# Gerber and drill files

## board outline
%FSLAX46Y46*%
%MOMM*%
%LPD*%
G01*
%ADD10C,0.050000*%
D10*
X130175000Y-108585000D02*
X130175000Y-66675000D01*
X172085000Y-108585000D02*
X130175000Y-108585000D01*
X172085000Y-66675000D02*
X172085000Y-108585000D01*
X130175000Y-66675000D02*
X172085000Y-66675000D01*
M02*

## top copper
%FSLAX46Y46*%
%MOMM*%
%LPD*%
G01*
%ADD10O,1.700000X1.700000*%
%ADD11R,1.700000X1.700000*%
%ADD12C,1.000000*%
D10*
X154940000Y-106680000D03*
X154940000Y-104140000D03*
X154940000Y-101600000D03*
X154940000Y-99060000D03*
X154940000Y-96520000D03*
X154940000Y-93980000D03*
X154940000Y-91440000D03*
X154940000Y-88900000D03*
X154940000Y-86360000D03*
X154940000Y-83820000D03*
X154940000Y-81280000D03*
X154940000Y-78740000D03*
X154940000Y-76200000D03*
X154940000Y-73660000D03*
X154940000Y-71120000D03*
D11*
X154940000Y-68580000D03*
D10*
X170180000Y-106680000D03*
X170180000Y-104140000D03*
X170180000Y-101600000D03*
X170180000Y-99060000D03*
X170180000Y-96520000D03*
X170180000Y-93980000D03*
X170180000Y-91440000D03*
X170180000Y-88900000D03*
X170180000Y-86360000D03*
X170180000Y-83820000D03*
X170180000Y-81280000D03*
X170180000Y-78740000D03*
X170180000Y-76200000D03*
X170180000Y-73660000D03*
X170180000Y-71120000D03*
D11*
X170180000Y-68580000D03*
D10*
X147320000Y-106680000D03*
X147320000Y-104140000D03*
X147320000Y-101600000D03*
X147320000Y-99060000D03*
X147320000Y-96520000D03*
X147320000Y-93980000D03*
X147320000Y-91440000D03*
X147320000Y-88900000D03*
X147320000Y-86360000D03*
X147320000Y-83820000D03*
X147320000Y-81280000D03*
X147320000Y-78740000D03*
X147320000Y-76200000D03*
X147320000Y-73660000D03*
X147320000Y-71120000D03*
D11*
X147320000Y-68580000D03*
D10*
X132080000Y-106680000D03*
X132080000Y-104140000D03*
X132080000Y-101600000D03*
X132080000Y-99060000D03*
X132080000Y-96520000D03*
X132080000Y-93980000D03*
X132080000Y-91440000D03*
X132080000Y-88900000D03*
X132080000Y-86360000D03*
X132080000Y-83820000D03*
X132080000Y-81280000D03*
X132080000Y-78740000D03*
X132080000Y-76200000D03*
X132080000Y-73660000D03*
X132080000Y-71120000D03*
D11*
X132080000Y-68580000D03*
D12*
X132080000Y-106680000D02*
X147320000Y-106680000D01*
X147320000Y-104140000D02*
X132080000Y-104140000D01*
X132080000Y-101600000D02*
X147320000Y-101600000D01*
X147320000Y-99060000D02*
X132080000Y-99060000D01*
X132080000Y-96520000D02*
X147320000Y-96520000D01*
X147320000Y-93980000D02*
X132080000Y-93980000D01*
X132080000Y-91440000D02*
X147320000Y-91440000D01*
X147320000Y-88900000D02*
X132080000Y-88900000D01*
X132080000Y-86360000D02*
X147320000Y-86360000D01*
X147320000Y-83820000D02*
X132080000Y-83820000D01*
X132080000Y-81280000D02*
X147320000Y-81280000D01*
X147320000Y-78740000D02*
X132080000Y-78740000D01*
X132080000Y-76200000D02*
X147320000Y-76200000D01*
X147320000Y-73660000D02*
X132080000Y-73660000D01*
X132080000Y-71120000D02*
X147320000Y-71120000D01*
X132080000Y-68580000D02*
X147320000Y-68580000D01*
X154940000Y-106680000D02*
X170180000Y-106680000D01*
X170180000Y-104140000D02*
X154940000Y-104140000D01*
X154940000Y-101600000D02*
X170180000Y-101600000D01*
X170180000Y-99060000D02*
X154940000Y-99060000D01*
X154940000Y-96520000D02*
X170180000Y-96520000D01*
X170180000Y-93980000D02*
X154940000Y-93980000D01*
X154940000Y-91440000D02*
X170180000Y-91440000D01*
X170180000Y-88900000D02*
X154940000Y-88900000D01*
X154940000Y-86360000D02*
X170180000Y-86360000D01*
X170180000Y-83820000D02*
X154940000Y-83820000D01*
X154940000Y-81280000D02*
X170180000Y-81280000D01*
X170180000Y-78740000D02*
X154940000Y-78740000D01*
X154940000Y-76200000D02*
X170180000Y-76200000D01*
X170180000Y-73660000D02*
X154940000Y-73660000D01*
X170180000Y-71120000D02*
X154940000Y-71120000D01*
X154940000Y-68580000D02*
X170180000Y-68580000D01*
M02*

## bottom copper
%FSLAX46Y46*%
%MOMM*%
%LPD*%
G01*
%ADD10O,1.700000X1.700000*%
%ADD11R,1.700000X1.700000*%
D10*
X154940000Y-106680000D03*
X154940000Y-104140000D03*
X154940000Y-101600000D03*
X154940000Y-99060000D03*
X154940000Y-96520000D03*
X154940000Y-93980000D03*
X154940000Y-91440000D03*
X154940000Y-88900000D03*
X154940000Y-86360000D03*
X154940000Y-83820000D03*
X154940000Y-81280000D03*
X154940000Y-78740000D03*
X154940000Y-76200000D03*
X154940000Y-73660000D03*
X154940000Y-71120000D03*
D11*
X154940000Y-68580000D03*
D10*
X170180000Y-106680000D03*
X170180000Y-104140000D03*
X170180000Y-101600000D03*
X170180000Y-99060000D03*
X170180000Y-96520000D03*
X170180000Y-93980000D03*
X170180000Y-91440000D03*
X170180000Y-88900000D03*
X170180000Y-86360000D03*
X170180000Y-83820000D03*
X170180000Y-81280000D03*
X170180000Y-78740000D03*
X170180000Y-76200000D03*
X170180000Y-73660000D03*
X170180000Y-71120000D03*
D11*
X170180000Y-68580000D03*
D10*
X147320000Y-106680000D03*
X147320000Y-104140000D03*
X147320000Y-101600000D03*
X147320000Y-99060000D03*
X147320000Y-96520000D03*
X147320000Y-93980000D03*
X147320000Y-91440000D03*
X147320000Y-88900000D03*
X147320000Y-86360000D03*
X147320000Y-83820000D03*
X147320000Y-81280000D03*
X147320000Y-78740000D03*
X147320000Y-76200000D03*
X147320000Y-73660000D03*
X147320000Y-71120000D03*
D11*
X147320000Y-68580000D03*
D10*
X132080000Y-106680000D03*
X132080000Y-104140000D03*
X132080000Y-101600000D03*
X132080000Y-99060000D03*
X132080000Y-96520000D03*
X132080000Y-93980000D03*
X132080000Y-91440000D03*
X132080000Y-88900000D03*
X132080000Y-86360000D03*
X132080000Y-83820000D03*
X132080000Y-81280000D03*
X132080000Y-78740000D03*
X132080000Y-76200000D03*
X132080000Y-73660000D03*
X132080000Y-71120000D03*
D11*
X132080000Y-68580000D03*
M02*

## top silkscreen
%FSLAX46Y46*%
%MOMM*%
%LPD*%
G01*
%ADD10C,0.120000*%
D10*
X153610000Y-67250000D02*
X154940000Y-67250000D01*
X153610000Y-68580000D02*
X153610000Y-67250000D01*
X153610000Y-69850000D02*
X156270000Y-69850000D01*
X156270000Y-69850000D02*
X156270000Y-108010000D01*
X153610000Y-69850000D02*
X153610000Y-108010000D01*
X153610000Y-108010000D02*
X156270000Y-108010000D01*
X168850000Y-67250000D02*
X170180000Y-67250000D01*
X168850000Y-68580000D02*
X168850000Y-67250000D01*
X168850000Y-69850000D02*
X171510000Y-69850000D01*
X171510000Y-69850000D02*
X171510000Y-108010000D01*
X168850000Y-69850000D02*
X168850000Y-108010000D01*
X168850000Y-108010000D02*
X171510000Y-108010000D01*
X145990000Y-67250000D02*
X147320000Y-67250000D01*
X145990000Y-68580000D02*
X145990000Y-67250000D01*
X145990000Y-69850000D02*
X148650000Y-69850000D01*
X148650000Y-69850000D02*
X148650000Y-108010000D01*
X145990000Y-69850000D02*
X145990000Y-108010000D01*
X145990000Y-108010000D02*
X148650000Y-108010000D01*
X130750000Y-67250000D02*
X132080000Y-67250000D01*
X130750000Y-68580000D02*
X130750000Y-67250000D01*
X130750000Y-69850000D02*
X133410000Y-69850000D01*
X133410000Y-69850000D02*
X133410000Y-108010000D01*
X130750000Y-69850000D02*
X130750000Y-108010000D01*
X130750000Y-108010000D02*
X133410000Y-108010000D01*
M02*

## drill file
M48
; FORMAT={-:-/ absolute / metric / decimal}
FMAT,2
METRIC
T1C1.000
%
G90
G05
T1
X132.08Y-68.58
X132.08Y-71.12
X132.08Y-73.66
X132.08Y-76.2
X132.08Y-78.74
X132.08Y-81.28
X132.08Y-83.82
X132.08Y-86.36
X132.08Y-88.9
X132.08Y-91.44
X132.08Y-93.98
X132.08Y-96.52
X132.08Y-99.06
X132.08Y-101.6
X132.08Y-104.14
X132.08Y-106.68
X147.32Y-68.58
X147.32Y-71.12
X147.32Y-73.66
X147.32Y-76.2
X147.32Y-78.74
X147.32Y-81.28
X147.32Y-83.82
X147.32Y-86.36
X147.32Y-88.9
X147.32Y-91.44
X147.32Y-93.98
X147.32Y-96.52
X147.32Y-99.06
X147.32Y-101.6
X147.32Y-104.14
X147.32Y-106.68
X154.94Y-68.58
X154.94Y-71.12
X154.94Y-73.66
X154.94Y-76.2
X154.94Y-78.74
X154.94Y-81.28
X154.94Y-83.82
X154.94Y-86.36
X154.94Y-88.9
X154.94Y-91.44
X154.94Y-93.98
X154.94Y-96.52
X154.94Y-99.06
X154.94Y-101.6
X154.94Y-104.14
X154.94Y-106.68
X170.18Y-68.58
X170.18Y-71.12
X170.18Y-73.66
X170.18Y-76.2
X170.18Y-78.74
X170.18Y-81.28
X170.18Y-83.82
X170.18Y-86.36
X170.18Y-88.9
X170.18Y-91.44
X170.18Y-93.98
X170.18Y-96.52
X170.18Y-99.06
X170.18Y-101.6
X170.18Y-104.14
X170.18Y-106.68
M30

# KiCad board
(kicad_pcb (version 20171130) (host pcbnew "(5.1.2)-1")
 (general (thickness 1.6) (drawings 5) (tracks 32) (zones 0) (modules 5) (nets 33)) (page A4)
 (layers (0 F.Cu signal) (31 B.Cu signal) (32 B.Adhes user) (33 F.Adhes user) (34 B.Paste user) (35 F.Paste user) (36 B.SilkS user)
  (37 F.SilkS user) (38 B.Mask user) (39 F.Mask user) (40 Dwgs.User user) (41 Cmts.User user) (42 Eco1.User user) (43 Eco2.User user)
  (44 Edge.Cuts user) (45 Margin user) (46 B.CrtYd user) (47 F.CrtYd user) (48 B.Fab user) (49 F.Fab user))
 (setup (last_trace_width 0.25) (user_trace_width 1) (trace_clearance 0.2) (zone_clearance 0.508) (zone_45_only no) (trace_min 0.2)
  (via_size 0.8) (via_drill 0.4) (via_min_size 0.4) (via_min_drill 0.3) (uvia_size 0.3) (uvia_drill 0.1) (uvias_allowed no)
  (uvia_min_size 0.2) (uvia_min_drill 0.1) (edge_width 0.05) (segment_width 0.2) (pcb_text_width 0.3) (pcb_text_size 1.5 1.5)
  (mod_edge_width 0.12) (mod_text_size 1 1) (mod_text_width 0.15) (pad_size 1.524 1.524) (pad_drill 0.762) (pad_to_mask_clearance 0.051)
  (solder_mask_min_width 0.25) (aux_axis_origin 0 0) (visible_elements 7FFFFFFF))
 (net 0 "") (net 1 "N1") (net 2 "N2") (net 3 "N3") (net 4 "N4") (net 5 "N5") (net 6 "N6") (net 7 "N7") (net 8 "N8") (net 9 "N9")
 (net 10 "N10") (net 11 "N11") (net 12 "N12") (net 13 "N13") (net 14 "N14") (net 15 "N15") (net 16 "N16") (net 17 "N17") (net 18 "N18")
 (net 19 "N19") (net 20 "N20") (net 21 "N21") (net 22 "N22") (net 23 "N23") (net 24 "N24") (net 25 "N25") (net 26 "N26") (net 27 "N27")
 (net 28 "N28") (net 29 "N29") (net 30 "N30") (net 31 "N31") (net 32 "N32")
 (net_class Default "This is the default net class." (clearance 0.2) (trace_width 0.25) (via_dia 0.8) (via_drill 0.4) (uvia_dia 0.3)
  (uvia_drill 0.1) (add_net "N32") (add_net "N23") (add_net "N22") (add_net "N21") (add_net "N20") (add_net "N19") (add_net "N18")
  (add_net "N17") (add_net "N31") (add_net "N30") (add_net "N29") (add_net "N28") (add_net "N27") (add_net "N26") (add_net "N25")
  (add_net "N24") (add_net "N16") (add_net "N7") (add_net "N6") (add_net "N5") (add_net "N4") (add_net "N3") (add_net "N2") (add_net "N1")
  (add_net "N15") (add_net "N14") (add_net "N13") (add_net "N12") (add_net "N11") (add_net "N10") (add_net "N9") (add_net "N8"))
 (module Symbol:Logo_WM (layer B.Cu) (at 161.925 83.82 90)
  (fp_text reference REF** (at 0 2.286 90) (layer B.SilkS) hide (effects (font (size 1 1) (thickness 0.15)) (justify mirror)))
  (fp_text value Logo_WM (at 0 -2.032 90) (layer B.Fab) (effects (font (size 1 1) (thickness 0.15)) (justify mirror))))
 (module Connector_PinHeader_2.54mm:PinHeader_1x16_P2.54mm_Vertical (layer F.Cu) (at 154.94 68.58)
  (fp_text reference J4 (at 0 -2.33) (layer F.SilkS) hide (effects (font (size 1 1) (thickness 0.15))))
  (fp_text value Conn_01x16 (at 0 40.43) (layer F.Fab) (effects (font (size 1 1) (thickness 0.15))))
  (fp_line (start -1.33 -1.33) (end 0 -1.33) (layer F.SilkS) (width 0.12))
  (fp_line (start -1.33 0) (end -1.33 -1.33) (layer F.SilkS) (width 0.12))
  (fp_line (start -1.33 1.27) (end 1.33 1.27) (layer F.SilkS) (width 0.12))
  (fp_line (start 1.33 1.27) (end 1.33 39.43) (layer F.SilkS) (width 0.12))
  (fp_line (start -1.33 1.27) (end -1.33 39.43) (layer F.SilkS) (width 0.12))
  (fp_line (start -1.33 39.43) (end 1.33 39.43) (layer F.SilkS) (width 0.12))
  (pad 16 thru_hole oval (at 0 38.1) (size 1.7 1.7) (drill 1) (layers *.Cu *.Mask) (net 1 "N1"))
  (pad 15 thru_hole oval (at 0 35.56) (size 1.7 1.7) (drill 1) (layers *.Cu *.Mask) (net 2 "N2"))
  (pad 14 thru_hole oval (at 0 33.02) (size 1.7 1.7) (drill 1) (layers *.Cu *.Mask) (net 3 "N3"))
  (pad 13 thru_hole oval (at 0 30.48) (size 1.7 1.7) (drill 1) (layers *.Cu *.Mask) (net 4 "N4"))
  (pad 12 thru_hole oval (at 0 27.94) (size 1.7 1.7) (drill 1) (layers *.Cu *.Mask) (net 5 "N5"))
  (pad 11 thru_hole oval (at 0 25.4) (size 1.7 1.7) (drill 1) (layers *.Cu *.Mask) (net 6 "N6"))
  (pad 10 thru_hole oval (at 0 22.86) (size 1.7 1.7) (drill 1) (layers *.Cu *.Mask) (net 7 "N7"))
  (pad 9 thru_hole oval (at 0 20.32) (size 1.7 1.7) (drill 1) (layers *.Cu *.Mask) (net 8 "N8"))
  (pad 8 thru_hole oval (at 0 17.78) (size 1.7 1.7) (drill 1) (layers *.Cu *.Mask) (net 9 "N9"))
  (pad 7 thru_hole oval (at 0 15.24) (size 1.7 1.7) (drill 1) (layers *.Cu *.Mask) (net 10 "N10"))
  (pad 6 thru_hole oval (at 0 12.7) (size 1.7 1.7) (drill 1) (layers *.Cu *.Mask) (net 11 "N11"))
  (pad 5 thru_hole oval (at 0 10.16) (size 1.7 1.7) (drill 1) (layers *.Cu *.Mask) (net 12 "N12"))
  (pad 4 thru_hole oval (at 0 7.62) (size 1.7 1.7) (drill 1) (layers *.Cu *.Mask) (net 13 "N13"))
  (pad 3 thru_hole oval (at 0 5.08) (size 1.7 1.7) (drill 1) (layers *.Cu *.Mask) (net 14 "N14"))
  (pad 2 thru_hole oval (at 0 2.54) (size 1.7 1.7) (drill 1) (layers *.Cu *.Mask) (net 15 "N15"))
  (pad 1 thru_hole rect (at 0 0) (size 1.7 1.7) (drill 1) (layers *.Cu *.Mask) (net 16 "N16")))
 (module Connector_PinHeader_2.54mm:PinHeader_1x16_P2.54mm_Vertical (layer F.Cu) (at 170.18 68.58)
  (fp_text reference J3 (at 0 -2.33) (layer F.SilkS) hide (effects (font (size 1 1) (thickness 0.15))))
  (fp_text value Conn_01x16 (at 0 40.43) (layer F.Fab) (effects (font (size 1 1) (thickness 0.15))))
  (fp_line (start -1.33 -1.33) (end 0 -1.33) (layer F.SilkS) (width 0.12))
  (fp_line (start -1.33 0) (end -1.33 -1.33) (layer F.SilkS) (width 0.12))
  (fp_line (start -1.33 1.27) (end 1.33 1.27) (layer F.SilkS) (width 0.12))
  (fp_line (start 1.33 1.27) (end 1.33 39.43) (layer F.SilkS) (width 0.12))
  (fp_line (start -1.33 1.27) (end -1.33 39.43) (layer F.SilkS) (width 0.12))
  (fp_line (start -1.33 39.43) (end 1.33 39.43) (layer F.SilkS) (width 0.12))
  (pad 16 thru_hole oval (at 0 38.1) (size 1.7 1.7) (drill 1) (layers *.Cu *.Mask) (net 1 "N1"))
  (pad 15 thru_hole oval (at 0 35.56) (size 1.7 1.7) (drill 1) (layers *.Cu *.Mask) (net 2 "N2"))
  (pad 14 thru_hole oval (at 0 33.02) (size 1.7 1.7) (drill 1) (layers *.Cu *.Mask) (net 3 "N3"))
  (pad 13 thru_hole oval (at 0 30.48) (size 1.7 1.7) (drill 1) (layers *.Cu *.Mask) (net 4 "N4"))
  (pad 12 thru_hole oval (at 0 27.94) (size 1.7 1.7) (drill 1) (layers *.Cu *.Mask) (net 5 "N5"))
  (pad 11 thru_hole oval (at 0 25.4) (size 1.7 1.7) (drill 1) (layers *.Cu *.Mask) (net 6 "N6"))
  (pad 10 thru_hole oval (at 0 22.86) (size 1.7 1.7) (drill 1) (layers *.Cu *.Mask) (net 7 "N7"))
  (pad 9 thru_hole oval (at 0 20.32) (size 1.7 1.7) (drill 1) (layers *.Cu *.Mask) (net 8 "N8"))
  (pad 8 thru_hole oval (at 0 17.78) (size 1.7 1.7) (drill 1) (layers *.Cu *.Mask) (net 9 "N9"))
  (pad 7 thru_hole oval (at 0 15.24) (size 1.7 1.7) (drill 1) (layers *.Cu *.Mask) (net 10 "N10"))
  (pad 6 thru_hole oval (at 0 12.7) (size 1.7 1.7) (drill 1) (layers *.Cu *.Mask) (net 11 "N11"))
  (pad 5 thru_hole oval (at 0 10.16) (size 1.7 1.7) (drill 1) (layers *.Cu *.Mask) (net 12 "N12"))
  (pad 4 thru_hole oval (at 0 7.62) (size 1.7 1.7) (drill 1) (layers *.Cu *.Mask) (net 13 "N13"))
  (pad 3 thru_hole oval (at 0 5.08) (size 1.7 1.7) (drill 1) (layers *.Cu *.Mask) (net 14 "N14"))
  (pad 2 thru_hole oval (at 0 2.54) (size 1.7 1.7) (drill 1) (layers *.Cu *.Mask) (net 15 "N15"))
  (pad 1 thru_hole rect (at 0 0) (size 1.7 1.7) (drill 1) (layers *.Cu *.Mask) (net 16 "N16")))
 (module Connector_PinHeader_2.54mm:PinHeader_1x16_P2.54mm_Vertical (layer F.Cu) (at 147.32 68.58)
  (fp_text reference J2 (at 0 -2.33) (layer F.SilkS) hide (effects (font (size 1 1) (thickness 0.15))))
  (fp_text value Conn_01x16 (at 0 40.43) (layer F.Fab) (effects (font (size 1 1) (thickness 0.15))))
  (fp_line (start -1.33 -1.33) (end 0 -1.33) (layer F.SilkS) (width 0.12))
  (fp_line (start -1.33 0) (end -1.33 -1.33) (layer F.SilkS) (width 0.12))
  (fp_line (start -1.33 1.27) (end 1.33 1.27) (layer F.SilkS) (width 0.12))
  (fp_line (start 1.33 1.27) (end 1.33 39.43) (layer F.SilkS) (width 0.12))
  (fp_line (start -1.33 1.27) (end -1.33 39.43) (layer F.SilkS) (width 0.12))
  (fp_line (start -1.33 39.43) (end 1.33 39.43) (layer F.SilkS) (width 0.12))
  (pad 16 thru_hole oval (at 0 38.1) (size 1.7 1.7) (drill 1) (layers *.Cu *.Mask) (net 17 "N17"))
  (pad 15 thru_hole oval (at 0 35.56) (size 1.7 1.7) (drill 1) (layers *.Cu *.Mask) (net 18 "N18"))
  (pad 14 thru_hole oval (at 0 33.02) (size 1.7 1.7) (drill 1) (layers *.Cu *.Mask) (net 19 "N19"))
  (pad 13 thru_hole oval (at 0 30.48) (size 1.7 1.7) (drill 1) (layers *.Cu *.Mask) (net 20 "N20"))
  (pad 12 thru_hole oval (at 0 27.94) (size 1.7 1.7) (drill 1) (layers *.Cu *.Mask) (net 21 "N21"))
  (pad 11 thru_hole oval (at 0 25.4) (size 1.7 1.7) (drill 1) (layers *.Cu *.Mask) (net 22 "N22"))
  (pad 10 thru_hole oval (at 0 22.86) (size 1.7 1.7) (drill 1) (layers *.Cu *.Mask) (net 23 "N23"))
  (pad 9 thru_hole oval (at 0 20.32) (size 1.7 1.7) (drill 1) (layers *.Cu *.Mask) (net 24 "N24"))
  (pad 8 thru_hole oval (at 0 17.78) (size 1.7 1.7) (drill 1) (layers *.Cu *.Mask) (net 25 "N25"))
  (pad 7 thru_hole oval (at 0 15.24) (size 1.7 1.7) (drill 1) (layers *.Cu *.Mask) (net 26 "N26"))
  (pad 6 thru_hole oval (at 0 12.7) (size 1.7 1.7) (drill 1) (layers *.Cu *.Mask) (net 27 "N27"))
  (pad 5 thru_hole oval (at 0 10.16) (size 1.7 1.7) (drill 1) (layers *.Cu *.Mask) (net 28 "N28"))
  (pad 4 thru_hole oval (at 0 7.62) (size 1.7 1.7) (drill 1) (layers *.Cu *.Mask) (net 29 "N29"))
  (pad 3 thru_hole oval (at 0 5.08) (size 1.7 1.7) (drill 1) (layers *.Cu *.Mask) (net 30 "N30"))
  (pad 2 thru_hole oval (at 0 2.54) (size 1.7 1.7) (drill 1) (layers *.Cu *.Mask) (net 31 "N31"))
  (pad 1 thru_hole rect (at 0 0) (size 1.7 1.7) (drill 1) (layers *.Cu *.Mask) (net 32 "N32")))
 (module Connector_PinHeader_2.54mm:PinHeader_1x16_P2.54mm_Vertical (layer F.Cu) (at 132.08 68.58)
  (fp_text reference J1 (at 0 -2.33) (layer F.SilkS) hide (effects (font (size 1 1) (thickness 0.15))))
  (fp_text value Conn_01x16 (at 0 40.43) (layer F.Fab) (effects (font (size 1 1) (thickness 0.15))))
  (fp_line (start -1.33 -1.33) (end 0 -1.33) (layer F.SilkS) (width 0.12))
  (fp_line (start -1.33 0) (end -1.33 -1.33) (layer F.SilkS) (width 0.12))
  (fp_line (start -1.33 1.27) (end 1.33 1.27) (layer F.SilkS) (width 0.12))
  (fp_line (start 1.33 1.27) (end 1.33 39.43) (layer F.SilkS) (width 0.12))
  (fp_line (start -1.33 1.27) (end -1.33 39.43) (layer F.SilkS) (width 0.12))
  (fp_line (start -1.33 39.43) (end 1.33 39.43) (layer F.SilkS) (width 0.12))
  (pad 16 thru_hole oval (at 0 38.1) (size 1.7 1.7) (drill 1) (layers *.Cu *.Mask) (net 17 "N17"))
  (pad 15 thru_hole oval (at 0 35.56) (size 1.7 1.7) (drill 1) (layers *.Cu *.Mask) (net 18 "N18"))
  (pad 14 thru_hole oval (at 0 33.02) (size 1.7 1.7) (drill 1) (layers *.Cu *.Mask) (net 19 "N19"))
  (pad 13 thru_hole oval (at 0 30.48) (size 1.7 1.7) (drill 1) (layers *.Cu *.Mask) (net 20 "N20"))
  (pad 12 thru_hole oval (at 0 27.94) (size 1.7 1.7) (drill 1) (layers *.Cu *.Mask) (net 21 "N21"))
  (pad 11 thru_hole oval (at 0 25.4) (size 1.7 1.7) (drill 1) (layers *.Cu *.Mask) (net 22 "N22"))
  (pad 10 thru_hole oval (at 0 22.86) (size 1.7 1.7) (drill 1) (layers *.Cu *.Mask) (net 23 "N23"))
  (pad 9 thru_hole oval (at 0 20.32) (size 1.7 1.7) (drill 1) (layers *.Cu *.Mask) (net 24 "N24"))
  (pad 8 thru_hole oval (at 0 17.78) (size 1.7 1.7) (drill 1) (layers *.Cu *.Mask) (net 25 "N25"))
  (pad 7 thru_hole oval (at 0 15.24) (size 1.7 1.7) (drill 1) (layers *.Cu *.Mask) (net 26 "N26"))
  (pad 6 thru_hole oval (at 0 12.7) (size 1.7 1.7) (drill 1) (layers *.Cu *.Mask) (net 27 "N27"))
  (pad 5 thru_hole oval (at 0 10.16) (size 1.7 1.7) (drill 1) (layers *.Cu *.Mask) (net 28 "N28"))
  (pad 4 thru_hole oval (at 0 7.62) (size 1.7 1.7) (drill 1) (layers *.Cu *.Mask) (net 29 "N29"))
  (pad 3 thru_hole oval (at 0 5.08) (size 1.7 1.7) (drill 1) (layers *.Cu *.Mask) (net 30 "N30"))
  (pad 2 thru_hole oval (at 0 2.54) (size 1.7 1.7) (drill 1) (layers *.Cu *.Mask) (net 31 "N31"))
  (pad 1 thru_hole rect (at 0 0) (size 1.7 1.7) (drill 1) (layers *.Cu *.Mask) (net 32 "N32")))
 (gr_line (start 130.175 108.585) (end 130.175 66.675) (layer Edge.Cuts) (width 0.05))
 (gr_line (start 172.085 108.585) (end 130.175 108.585) (layer Edge.Cuts) (width 0.05))
 (gr_line (start 172.085 66.675) (end 172.085 108.585) (layer Edge.Cuts) (width 0.05))
 (gr_line (start 130.175 66.675) (end 172.085 66.675) (layer Edge.Cuts) (width 0.05))
 (segment (start 132.08 106.68) (end 147.32 106.68) (width 1) (layer F.Cu) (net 17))
 (segment (start 147.32 104.14) (end 132.08 104.14) (width 1) (layer F.Cu) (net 18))
 (segment (start 132.08 101.6) (end 147.32 101.6) (width 1) (layer F.Cu) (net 19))
 (segment (start 147.32 99.06) (end 132.08 99.06) (width 1) (layer F.Cu) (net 20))
 (segment (start 132.08 96.52) (end 147.32 96.52) (width 1) (layer F.Cu) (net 21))
 (segment (start 147.32 93.98) (end 132.08 93.98) (width 1) (layer F.Cu) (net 22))
 (segment (start 132.08 91.44) (end 147.32 91.44) (width 1) (layer F.Cu) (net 23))
 (segment (start 147.32 88.9) (end 132.08 88.9) (width 1) (layer F.Cu) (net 24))
 (segment (start 132.08 86.36) (end 147.32 86.36) (width 1) (layer F.Cu) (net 25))
 (segment (start 147.32 83.82) (end 132.08 83.82) (width 1) (layer F.Cu) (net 26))
 (segment (start 132.08 81.28) (end 147.32 81.28) (width 1) (layer F.Cu) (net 27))
 (segment (start 147.32 78.74) (end 132.08 78.74) (width 1) (layer F.Cu) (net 28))
 (segment (start 132.08 76.2) (end 147.32 76.2) (width 1) (layer F.Cu) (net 29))
 (segment (start 147.32 73.66) (end 132.08 73.66) (width 1) (layer F.Cu) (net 30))
 (segment (start 132.08 71.12) (end 147.32 71.12) (width 1) (layer F.Cu) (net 31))
 (segment (start 132.08 68.58) (end 147.32 68.58) (width 1) (layer F.Cu) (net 32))
 (segment (start 154.94 106.68) (end 170.18 106.68) (width 1) (layer F.Cu) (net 1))
 (segment (start 170.18 104.14) (end 154.94 104.14) (width 1) (layer F.Cu) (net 2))
 (segment (start 154.94 101.6) (end 170.18 101.6) (width 1) (layer F.Cu) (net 3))
 (segment (start 170.18 99.06) (end 154.94 99.06) (width 1) (layer F.Cu) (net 4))
 (segment (start 154.94 96.52) (end 170.18 96.52) (width 1) (layer F.Cu) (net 5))
 (segment (start 170.18 93.98) (end 154.94 93.98) (width 1) (layer F.Cu) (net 6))
 (segment (start 154.94 91.44) (end 170.18 91.44) (width 1) (layer F.Cu) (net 7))
 (segment (start 170.18 88.9) (end 154.94 88.9) (width 1) (layer F.Cu) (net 8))
 (segment (start 154.94 86.36) (end 170.18 86.36) (width 1) (layer F.Cu) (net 9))
 (segment (start 170.18 83.82) (end 154.94 83.82) (width 1) (layer F.Cu) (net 10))
 (segment (start 154.94 81.28) (end 170.18 81.28) (width 1) (layer F.Cu) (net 11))
 (segment (start 170.18 78.74) (end 154.94 78.74) (width 1) (layer F.Cu) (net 12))
 (segment (start 154.94 76.2) (end 170.18 76.2) (width 1) (layer F.Cu) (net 13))
 (segment (start 170.18 73.66) (end 154.94 73.66) (width 1) (layer F.Cu) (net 14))
 (segment (start 170.18 71.12) (end 154.94 71.12) (width 1) (layer F.Cu) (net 15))
 (segment (start 154.94 68.58) (end 170.18 68.58) (width 1) (layer F.Cu) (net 16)))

